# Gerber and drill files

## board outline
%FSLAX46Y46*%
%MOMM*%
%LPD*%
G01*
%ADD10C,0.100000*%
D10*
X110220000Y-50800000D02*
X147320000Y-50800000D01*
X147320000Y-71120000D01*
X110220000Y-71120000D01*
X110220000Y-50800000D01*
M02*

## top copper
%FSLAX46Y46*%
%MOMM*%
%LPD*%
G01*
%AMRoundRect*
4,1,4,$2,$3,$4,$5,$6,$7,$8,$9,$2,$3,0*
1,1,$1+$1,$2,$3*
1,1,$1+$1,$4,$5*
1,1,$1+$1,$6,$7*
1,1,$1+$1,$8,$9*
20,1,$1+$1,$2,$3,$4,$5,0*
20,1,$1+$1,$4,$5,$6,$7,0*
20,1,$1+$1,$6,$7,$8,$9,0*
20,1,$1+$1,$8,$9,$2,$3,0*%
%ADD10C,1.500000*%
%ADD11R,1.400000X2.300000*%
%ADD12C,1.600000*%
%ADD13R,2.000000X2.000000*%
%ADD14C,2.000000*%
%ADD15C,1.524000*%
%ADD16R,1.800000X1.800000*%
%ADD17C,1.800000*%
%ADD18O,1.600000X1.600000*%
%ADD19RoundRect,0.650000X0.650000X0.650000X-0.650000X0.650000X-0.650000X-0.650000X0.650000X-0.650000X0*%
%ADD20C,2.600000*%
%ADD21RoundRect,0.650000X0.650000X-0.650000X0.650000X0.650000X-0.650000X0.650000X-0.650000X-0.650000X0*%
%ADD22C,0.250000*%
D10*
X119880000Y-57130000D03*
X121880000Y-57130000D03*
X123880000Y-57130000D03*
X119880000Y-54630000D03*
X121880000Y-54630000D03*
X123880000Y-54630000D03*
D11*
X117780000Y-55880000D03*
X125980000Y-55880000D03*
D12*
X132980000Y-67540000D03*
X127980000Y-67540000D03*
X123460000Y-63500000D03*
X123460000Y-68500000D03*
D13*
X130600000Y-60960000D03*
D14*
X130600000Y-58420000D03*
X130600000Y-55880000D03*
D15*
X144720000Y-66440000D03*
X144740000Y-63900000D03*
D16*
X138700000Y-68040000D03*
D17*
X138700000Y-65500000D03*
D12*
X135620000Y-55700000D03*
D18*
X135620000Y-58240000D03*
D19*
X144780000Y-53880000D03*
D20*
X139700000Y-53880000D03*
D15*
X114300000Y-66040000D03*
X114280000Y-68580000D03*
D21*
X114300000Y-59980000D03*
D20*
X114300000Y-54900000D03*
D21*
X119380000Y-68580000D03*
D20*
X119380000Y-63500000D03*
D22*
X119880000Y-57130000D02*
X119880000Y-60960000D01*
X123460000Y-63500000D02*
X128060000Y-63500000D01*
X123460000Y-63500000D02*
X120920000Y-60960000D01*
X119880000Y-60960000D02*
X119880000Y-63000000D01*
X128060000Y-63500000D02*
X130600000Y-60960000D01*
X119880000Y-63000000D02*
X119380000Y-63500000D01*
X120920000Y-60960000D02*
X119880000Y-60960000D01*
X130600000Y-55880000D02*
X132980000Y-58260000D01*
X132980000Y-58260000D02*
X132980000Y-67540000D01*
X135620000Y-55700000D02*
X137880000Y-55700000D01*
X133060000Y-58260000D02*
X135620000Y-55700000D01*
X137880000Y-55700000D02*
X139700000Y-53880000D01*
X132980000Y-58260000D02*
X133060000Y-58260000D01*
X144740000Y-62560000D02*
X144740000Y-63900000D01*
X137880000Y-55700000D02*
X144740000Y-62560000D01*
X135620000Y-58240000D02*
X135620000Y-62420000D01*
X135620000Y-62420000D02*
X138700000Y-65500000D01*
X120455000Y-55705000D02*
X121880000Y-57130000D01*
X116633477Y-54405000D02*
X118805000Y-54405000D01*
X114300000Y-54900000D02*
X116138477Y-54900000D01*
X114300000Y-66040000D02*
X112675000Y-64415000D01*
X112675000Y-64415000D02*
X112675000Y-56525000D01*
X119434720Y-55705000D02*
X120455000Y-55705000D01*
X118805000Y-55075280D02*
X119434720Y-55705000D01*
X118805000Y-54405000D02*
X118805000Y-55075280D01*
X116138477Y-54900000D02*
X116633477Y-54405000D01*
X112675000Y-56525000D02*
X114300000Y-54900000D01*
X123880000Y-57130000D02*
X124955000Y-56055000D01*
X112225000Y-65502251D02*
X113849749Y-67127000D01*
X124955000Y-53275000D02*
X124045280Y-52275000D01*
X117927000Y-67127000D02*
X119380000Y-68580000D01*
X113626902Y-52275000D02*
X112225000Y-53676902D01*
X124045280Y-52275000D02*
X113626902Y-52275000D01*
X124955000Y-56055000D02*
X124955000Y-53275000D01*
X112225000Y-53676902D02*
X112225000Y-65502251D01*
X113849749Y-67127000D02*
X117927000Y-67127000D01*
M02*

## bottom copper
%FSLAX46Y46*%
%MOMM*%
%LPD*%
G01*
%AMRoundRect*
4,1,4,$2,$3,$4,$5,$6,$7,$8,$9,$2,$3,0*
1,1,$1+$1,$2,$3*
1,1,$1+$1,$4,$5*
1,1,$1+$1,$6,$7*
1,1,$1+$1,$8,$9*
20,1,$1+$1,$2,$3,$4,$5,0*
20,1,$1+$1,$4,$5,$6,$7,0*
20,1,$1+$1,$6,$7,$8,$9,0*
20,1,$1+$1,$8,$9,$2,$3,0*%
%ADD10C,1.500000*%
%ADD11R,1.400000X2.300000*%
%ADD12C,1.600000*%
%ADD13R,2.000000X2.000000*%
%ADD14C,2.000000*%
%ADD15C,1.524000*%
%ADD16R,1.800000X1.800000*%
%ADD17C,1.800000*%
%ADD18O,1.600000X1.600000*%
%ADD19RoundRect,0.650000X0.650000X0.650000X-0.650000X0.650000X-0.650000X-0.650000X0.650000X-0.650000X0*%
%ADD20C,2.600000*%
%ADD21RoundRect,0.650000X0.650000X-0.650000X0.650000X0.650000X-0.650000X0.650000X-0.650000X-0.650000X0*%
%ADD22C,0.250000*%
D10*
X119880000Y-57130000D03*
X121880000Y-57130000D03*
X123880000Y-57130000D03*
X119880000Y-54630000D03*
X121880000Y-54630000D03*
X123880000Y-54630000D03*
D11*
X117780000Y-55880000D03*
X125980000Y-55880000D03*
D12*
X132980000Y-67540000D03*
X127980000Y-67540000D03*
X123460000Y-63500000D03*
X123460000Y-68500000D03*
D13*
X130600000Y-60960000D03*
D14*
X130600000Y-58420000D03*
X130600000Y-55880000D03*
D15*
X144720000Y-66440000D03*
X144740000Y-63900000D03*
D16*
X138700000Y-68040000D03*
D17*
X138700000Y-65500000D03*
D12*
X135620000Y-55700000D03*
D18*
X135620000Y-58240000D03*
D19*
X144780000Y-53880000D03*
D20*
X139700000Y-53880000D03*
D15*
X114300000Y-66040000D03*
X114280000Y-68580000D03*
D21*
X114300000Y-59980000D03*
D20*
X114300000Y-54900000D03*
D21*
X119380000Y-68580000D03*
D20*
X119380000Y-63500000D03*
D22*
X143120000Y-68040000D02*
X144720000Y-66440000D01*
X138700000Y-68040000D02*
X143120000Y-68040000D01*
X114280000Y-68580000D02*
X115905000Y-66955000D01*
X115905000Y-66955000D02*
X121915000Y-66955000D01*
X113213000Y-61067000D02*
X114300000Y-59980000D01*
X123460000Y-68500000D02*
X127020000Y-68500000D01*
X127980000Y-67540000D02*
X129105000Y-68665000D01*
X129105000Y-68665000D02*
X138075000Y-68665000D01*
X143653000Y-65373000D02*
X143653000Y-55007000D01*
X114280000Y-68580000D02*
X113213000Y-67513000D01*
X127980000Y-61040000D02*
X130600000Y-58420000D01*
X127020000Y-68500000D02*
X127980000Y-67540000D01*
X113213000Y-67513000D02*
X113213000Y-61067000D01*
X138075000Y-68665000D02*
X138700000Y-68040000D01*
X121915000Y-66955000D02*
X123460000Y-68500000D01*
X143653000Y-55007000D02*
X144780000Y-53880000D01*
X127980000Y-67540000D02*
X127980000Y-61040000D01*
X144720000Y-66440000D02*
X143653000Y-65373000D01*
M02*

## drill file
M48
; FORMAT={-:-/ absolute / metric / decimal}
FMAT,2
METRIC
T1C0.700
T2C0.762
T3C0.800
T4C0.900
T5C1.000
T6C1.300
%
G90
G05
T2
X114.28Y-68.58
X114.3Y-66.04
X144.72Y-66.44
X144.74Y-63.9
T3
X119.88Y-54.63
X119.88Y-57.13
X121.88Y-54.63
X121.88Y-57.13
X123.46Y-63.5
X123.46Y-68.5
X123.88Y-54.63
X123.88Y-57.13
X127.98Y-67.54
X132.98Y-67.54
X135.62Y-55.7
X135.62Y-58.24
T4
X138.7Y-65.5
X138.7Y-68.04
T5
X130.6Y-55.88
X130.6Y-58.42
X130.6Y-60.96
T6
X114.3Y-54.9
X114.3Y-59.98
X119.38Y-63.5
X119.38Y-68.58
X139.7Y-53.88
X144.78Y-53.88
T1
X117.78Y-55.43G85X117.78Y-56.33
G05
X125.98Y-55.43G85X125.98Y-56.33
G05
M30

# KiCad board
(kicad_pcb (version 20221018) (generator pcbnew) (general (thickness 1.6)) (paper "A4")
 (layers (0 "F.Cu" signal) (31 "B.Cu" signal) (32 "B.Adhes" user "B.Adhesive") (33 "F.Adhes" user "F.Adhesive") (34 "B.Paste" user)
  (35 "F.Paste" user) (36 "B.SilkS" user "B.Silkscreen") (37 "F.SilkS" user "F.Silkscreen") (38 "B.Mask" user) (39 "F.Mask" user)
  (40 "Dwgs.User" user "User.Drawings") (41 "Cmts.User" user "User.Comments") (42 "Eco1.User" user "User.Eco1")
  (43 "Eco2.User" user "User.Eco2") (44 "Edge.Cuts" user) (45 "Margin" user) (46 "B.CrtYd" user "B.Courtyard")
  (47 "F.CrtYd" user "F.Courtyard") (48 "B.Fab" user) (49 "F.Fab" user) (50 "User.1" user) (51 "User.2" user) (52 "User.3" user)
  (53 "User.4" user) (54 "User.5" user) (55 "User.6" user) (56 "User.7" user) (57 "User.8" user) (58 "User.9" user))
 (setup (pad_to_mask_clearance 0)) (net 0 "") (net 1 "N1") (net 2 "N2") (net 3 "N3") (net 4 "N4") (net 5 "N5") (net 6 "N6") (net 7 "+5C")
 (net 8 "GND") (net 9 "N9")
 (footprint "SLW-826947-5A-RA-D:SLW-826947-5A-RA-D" (layer "F.Cu") (at 121.88 55.88)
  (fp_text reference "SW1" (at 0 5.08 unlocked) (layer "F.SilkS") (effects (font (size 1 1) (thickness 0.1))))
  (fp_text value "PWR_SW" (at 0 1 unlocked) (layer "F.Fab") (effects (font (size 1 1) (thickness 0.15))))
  (pad "1" thru_hole circle (at -2 1.25) (size 1.5 1.5) (drill 0.8) (layers "*.Cu" "*.Mask") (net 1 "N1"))
  (pad "2" thru_hole circle (at 0 1.25) (size 1.5 1.5) (drill 0.8) (layers "*.Cu" "*.Mask") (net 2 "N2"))
  (pad "3" thru_hole circle (at 2 1.25) (size 1.5 1.5) (drill 0.8) (layers "*.Cu" "*.Mask") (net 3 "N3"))
  (pad "4" thru_hole circle (at -2 -1.25) (size 1.5 1.5) (drill 0.8) (layers "*.Cu" "*.Mask") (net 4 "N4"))
  (pad "5" thru_hole circle (at 0 -1.25) (size 1.5 1.5) (drill 0.8) (layers "*.Cu" "*.Mask") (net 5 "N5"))
  (pad "6" thru_hole circle (at 2 -1.25) (size 1.5 1.5) (drill 0.8) (layers "*.Cu" "*.Mask") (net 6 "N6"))
  (pad "7" thru_hole rect (at -4.1 0) (size 1.4 2.3) (drill oval 0.7 1.6) (layers "*.Cu" "*.Mask"))
  (pad "8" thru_hole rect (at 4.1 0) (size 1.4 2.3) (drill oval 0.7 1.6) (layers "*.Cu" "*.Mask")))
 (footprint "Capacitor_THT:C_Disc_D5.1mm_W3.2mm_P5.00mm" (layer "F.Cu") (at 132.98 67.54 180)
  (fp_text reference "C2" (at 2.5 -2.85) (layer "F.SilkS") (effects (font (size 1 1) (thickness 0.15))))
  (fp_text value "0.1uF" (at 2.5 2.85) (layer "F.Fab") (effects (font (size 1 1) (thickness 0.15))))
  (pad "1" thru_hole circle (at 0 0 180) (size 1.6 1.6) (drill 0.8) (layers "*.Cu" "*.Mask") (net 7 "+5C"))
  (pad "2" thru_hole circle (at 5 0 180) (size 1.6 1.6) (drill 0.8) (layers "*.Cu" "*.Mask") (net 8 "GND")))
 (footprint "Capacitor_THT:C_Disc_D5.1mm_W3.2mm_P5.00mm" (layer "F.Cu") (at 123.46 63.5 -90)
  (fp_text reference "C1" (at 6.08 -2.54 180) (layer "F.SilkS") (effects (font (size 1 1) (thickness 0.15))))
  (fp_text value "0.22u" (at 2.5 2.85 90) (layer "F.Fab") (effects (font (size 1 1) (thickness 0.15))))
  (pad "1" thru_hole circle (at 0 0 270) (size 1.6 1.6) (drill 0.8) (layers "*.Cu" "*.Mask") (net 1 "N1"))
  (pad "2" thru_hole circle (at 5 0 270) (size 1.6 1.6) (drill 0.8) (layers "*.Cu" "*.Mask") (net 8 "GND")))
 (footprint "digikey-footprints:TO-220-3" (layer "F.Cu") (at 130.6 60.96 90)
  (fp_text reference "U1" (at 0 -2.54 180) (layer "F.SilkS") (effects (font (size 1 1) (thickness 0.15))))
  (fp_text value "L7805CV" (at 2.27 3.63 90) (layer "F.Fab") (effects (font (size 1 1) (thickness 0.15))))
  (pad "1" thru_hole rect (at 0 0 90) (size 2 2) (drill 1) (layers "*.Cu" "*.Mask") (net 1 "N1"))
  (pad "2" thru_hole circle (at 2.54 0 90) (size 2 2) (drill 1) (layers "*.Cu" "*.Mask") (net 8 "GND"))
  (pad "3" thru_hole circle (at 5.08 0 90) (size 2 2) (drill 1) (layers "*.Cu" "*.Mask") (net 7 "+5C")))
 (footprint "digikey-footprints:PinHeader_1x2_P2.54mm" (layer "F.Cu") (at 144.72 66.44 90)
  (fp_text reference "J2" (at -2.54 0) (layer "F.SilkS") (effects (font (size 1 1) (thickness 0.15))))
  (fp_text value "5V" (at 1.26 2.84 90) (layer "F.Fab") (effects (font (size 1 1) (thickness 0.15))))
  (pad "1" thru_hole circle (at 0 0 90) (size 1.524 1.524) (drill 0.762) (layers "*.Cu" "*.Mask") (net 8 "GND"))
  (pad "2" thru_hole circle (at 2.54 0.02 90) (size 1.524 1.524) (drill 0.762) (layers "*.Cu" "*.Mask") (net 7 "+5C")))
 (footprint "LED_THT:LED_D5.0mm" (layer "F.Cu") (at 138.7 68.04 90)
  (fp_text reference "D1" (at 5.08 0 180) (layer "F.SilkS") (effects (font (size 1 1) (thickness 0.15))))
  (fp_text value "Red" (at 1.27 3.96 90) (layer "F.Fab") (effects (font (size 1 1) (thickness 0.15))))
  (pad "1" thru_hole rect (at 0 0 90) (size 1.8 1.8) (drill 0.9) (layers "*.Cu" "*.Mask") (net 8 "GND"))
  (pad "2" thru_hole circle (at 2.54 0 90) (size 1.8 1.8) (drill 0.9) (layers "*.Cu" "*.Mask") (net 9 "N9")))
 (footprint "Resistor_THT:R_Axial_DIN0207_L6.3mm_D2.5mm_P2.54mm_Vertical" (layer "F.Cu") (at 135.62 55.7 -90)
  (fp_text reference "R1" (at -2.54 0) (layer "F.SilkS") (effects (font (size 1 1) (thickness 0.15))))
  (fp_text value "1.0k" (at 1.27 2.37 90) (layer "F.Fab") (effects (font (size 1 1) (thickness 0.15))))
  (pad "1" thru_hole circle (at 0 0 270) (size 1.6 1.6) (drill 0.8) (layers "*.Cu" "*.Mask") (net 7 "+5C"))
  (pad "2" thru_hole oval (at 2.54 0 270) (size 1.6 1.6) (drill 0.8) (layers "*.Cu" "*.Mask") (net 9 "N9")))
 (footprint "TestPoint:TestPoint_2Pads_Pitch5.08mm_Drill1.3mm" (layer "F.Cu") (at 144.78 53.88 180)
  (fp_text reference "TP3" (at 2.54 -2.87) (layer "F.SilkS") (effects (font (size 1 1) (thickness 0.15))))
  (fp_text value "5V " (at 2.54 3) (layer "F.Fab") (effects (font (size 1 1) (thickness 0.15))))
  (pad "1" thru_hole roundrect (at 0 0 180) (size 2.6 2.6) (drill 1.3) (layers "*.Cu" "*.Mask") (roundrect_rratio 0.25) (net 8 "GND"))
  (pad "2" thru_hole circle (at 5.08 0 180) (size 2.6 2.6) (drill 1.3) (layers "*.Cu" "*.Mask") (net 7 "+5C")))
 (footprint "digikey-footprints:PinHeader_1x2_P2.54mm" (layer "F.Cu") (at 114.3 66.04 -90)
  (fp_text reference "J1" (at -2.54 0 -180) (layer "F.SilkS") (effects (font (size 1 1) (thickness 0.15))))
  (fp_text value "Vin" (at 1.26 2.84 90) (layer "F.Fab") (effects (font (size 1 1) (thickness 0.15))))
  (pad "1" thru_hole circle (at 0 0 270) (size 1.524 1.524) (drill 0.762) (layers "*.Cu" "*.Mask") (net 2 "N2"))
  (pad "2" thru_hole circle (at 2.54 0.02 270) (size 1.524 1.524) (drill 0.762) (layers "*.Cu" "*.Mask") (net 8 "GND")))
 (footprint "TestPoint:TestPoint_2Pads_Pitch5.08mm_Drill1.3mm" (layer "F.Cu") (at 114.3 59.98 90)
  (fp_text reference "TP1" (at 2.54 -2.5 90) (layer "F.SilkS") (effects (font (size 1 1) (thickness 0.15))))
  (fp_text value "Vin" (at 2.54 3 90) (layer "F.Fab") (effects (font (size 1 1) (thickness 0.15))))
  (pad "1" thru_hole roundrect (at 0 0 90) (size 2.6 2.6) (drill 1.3) (layers "*.Cu" "*.Mask") (roundrect_rratio 0.25) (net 8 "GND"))
  (pad "2" thru_hole circle (at 5.08 0 90) (size 2.6 2.6) (drill 1.3) (layers "*.Cu" "*.Mask") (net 2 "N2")))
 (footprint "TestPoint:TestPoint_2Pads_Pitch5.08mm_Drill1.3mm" (layer "F.Cu") (at 119.38 68.58 90)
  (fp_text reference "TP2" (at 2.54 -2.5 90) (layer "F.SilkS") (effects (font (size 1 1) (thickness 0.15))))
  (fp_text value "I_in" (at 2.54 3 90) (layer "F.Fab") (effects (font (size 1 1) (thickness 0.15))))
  (pad "1" thru_hole roundrect (at 0 0 90) (size 2.6 2.6) (drill 1.3) (layers "*.Cu" "*.Mask") (roundrect_rratio 0.25) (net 3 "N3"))
  (pad "2" thru_hole circle (at 5.08 0 90) (size 2.6 2.6) (drill 1.3) (layers "*.Cu" "*.Mask") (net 1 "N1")))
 (gr_rect (start 110.22 50.8) (end 147.32 71.12) (stroke (width 0.1) (type default)) (fill none) (layer "Edge.Cuts"))
 (segment (start 119.88 57.13) (end 119.88 60.96) (width 0.25) (layer "F.Cu") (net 1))
 (segment (start 123.46 63.5) (end 128.06 63.5) (width 0.25) (layer "F.Cu") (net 1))
 (segment (start 123.46 63.5) (end 120.92 60.96) (width 0.25) (layer "F.Cu") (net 1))
 (segment (start 119.88 60.96) (end 119.88 63) (width 0.25) (layer "F.Cu") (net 1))
 (segment (start 128.06 63.5) (end 130.6 60.96) (width 0.25) (layer "F.Cu") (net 1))
 (segment (start 119.88 63) (end 119.38 63.5) (width 0.25) (layer "F.Cu") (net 1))
 (segment (start 120.92 60.96) (end 119.88 60.96) (width 0.25) (layer "F.Cu") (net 1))
 (segment (start 143.12 68.04) (end 144.72 66.44) (width 0.25) (layer "B.Cu") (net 8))
 (segment (start 138.7 68.04) (end 143.12 68.04) (width 0.25) (layer "B.Cu") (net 8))
 (segment (start 114.28 68.58) (end 115.905 66.955) (width 0.25) (layer "B.Cu") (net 8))
 (segment (start 115.905 66.955) (end 121.915 66.955) (width 0.25) (layer "B.Cu") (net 8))
 (segment (start 113.213 61.067) (end 114.3 59.98) (width 0.25) (layer "B.Cu") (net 8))
 (segment (start 123.46 68.5) (end 127.02 68.5) (width 0.25) (layer "B.Cu") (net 8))
 (segment (start 127.98 67.54) (end 129.105 68.665) (width 0.25) (layer "B.Cu") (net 8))
 (segment (start 129.105 68.665) (end 138.075 68.665) (width 0.25) (layer "B.Cu") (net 8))
 (segment (start 143.653 65.373) (end 143.653 55.007) (width 0.25) (layer "B.Cu") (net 8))
 (segment (start 114.28 68.58) (end 113.213 67.513) (width 0.25) (layer "B.Cu") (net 8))
 (segment (start 127.98 61.04) (end 130.6 58.42) (width 0.25) (layer "B.Cu") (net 8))
 (segment (start 127.02 68.5) (end 127.98 67.54) (width 0.25) (layer "B.Cu") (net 8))
 (segment (start 113.213 67.513) (end 113.213 61.067) (width 0.25) (layer "B.Cu") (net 8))
 (segment (start 138.075 68.665) (end 138.7 68.04) (width 0.25) (layer "B.Cu") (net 8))
 (segment (start 121.915 66.955) (end 123.46 68.5) (width 0.25) (layer "B.Cu") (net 8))
 (segment (start 143.653 55.007) (end 144.78 53.88) (width 0.25) (layer "B.Cu") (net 8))
 (segment (start 127.98 67.54) (end 127.98 61.04) (width 0.25) (layer "B.Cu") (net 8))
 (segment (start 144.72 66.44) (end 143.653 65.373) (width 0.25) (layer "B.Cu") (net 8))
 (segment (start 130.6 55.88) (end 132.98 58.26) (width 0.25) (layer "F.Cu") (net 7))
 (segment (start 132.98 58.26) (end 132.98 67.54) (width 0.25) (layer "F.Cu") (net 7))
 (segment (start 135.62 55.7) (end 137.88 55.7) (width 0.25) (layer "F.Cu") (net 7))
 (segment (start 133.06 58.26) (end 135.62 55.7) (width 0.25) (layer "F.Cu") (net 7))
 (segment (start 137.88 55.7) (end 139.7 53.88) (width 0.25) (layer "F.Cu") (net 7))
 (segment (start 132.98 58.26) (end 133.06 58.26) (width 0.25) (layer "F.Cu") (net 7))
 (segment (start 144.74 62.56) (end 144.74 63.9) (width 0.25) (layer "F.Cu") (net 7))
 (segment (start 137.88 55.7) (end 144.74 62.56) (width 0.25) (layer "F.Cu") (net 7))
 (segment (start 135.62 58.24) (end 135.62 62.42) (width 0.25) (layer "F.Cu") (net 9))
 (segment (start 135.62 62.42) (end 138.7 65.5) (width 0.25) (layer "F.Cu") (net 9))
 (segment (start 120.455 55.705) (end 121.88 57.13) (width 0.25) (layer "F.Cu") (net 2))
 (segment (start 116.633477 54.405) (end 118.805 54.405) (width 0.25) (layer "F.Cu") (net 2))
 (segment (start 114.3 54.9) (end 116.138477 54.9) (width 0.25) (layer "F.Cu") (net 2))
 (segment (start 114.3 66.04) (end 112.675 64.415) (width 0.25) (layer "F.Cu") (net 2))
 (segment (start 112.675 64.415) (end 112.675 56.525) (width 0.25) (layer "F.Cu") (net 2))
 (segment (start 119.43472 55.705) (end 120.455 55.705) (width 0.25) (layer "F.Cu") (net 2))
 (segment (start 118.805 55.07528) (end 119.43472 55.705) (width 0.25) (layer "F.Cu") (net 2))
 (segment (start 118.805 54.405) (end 118.805 55.07528) (width 0.25) (layer "F.Cu") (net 2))
 (segment (start 116.138477 54.9) (end 116.633477 54.405) (width 0.25) (layer "F.Cu") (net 2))
 (segment (start 112.675 56.525) (end 114.3 54.9) (width 0.25) (layer "F.Cu") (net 2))
 (segment (start 123.88 57.13) (end 124.955 56.055) (width 0.25) (layer "F.Cu") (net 3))
 (segment (start 112.225 65.502251) (end 113.849749 67.127) (width 0.25) (layer "F.Cu") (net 3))
 (segment (start 124.955 53.275) (end 124.04528 52.275) (width 0.25) (layer "F.Cu") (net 3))
 (segment (start 117.927 67.127) (end 119.38 68.58) (width 0.25) (layer "F.Cu") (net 3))
 (segment (start 113.626902 52.275) (end 112.225 53.676902) (width 0.25) (layer "F.Cu") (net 3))
 (segment (start 124.04528 52.275) (end 113.626902 52.275) (width 0.25) (layer "F.Cu") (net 3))
 (segment (start 124.955 56.055) (end 124.955 53.275) (width 0.25) (layer "F.Cu") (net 3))
 (segment (start 112.225 53.676902) (end 112.225 65.502251) (width 0.25) (layer "F.Cu") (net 3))
 (segment (start 113.849749 67.127) (end 117.927 67.127) (width 0.25) (layer "F.Cu") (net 3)))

